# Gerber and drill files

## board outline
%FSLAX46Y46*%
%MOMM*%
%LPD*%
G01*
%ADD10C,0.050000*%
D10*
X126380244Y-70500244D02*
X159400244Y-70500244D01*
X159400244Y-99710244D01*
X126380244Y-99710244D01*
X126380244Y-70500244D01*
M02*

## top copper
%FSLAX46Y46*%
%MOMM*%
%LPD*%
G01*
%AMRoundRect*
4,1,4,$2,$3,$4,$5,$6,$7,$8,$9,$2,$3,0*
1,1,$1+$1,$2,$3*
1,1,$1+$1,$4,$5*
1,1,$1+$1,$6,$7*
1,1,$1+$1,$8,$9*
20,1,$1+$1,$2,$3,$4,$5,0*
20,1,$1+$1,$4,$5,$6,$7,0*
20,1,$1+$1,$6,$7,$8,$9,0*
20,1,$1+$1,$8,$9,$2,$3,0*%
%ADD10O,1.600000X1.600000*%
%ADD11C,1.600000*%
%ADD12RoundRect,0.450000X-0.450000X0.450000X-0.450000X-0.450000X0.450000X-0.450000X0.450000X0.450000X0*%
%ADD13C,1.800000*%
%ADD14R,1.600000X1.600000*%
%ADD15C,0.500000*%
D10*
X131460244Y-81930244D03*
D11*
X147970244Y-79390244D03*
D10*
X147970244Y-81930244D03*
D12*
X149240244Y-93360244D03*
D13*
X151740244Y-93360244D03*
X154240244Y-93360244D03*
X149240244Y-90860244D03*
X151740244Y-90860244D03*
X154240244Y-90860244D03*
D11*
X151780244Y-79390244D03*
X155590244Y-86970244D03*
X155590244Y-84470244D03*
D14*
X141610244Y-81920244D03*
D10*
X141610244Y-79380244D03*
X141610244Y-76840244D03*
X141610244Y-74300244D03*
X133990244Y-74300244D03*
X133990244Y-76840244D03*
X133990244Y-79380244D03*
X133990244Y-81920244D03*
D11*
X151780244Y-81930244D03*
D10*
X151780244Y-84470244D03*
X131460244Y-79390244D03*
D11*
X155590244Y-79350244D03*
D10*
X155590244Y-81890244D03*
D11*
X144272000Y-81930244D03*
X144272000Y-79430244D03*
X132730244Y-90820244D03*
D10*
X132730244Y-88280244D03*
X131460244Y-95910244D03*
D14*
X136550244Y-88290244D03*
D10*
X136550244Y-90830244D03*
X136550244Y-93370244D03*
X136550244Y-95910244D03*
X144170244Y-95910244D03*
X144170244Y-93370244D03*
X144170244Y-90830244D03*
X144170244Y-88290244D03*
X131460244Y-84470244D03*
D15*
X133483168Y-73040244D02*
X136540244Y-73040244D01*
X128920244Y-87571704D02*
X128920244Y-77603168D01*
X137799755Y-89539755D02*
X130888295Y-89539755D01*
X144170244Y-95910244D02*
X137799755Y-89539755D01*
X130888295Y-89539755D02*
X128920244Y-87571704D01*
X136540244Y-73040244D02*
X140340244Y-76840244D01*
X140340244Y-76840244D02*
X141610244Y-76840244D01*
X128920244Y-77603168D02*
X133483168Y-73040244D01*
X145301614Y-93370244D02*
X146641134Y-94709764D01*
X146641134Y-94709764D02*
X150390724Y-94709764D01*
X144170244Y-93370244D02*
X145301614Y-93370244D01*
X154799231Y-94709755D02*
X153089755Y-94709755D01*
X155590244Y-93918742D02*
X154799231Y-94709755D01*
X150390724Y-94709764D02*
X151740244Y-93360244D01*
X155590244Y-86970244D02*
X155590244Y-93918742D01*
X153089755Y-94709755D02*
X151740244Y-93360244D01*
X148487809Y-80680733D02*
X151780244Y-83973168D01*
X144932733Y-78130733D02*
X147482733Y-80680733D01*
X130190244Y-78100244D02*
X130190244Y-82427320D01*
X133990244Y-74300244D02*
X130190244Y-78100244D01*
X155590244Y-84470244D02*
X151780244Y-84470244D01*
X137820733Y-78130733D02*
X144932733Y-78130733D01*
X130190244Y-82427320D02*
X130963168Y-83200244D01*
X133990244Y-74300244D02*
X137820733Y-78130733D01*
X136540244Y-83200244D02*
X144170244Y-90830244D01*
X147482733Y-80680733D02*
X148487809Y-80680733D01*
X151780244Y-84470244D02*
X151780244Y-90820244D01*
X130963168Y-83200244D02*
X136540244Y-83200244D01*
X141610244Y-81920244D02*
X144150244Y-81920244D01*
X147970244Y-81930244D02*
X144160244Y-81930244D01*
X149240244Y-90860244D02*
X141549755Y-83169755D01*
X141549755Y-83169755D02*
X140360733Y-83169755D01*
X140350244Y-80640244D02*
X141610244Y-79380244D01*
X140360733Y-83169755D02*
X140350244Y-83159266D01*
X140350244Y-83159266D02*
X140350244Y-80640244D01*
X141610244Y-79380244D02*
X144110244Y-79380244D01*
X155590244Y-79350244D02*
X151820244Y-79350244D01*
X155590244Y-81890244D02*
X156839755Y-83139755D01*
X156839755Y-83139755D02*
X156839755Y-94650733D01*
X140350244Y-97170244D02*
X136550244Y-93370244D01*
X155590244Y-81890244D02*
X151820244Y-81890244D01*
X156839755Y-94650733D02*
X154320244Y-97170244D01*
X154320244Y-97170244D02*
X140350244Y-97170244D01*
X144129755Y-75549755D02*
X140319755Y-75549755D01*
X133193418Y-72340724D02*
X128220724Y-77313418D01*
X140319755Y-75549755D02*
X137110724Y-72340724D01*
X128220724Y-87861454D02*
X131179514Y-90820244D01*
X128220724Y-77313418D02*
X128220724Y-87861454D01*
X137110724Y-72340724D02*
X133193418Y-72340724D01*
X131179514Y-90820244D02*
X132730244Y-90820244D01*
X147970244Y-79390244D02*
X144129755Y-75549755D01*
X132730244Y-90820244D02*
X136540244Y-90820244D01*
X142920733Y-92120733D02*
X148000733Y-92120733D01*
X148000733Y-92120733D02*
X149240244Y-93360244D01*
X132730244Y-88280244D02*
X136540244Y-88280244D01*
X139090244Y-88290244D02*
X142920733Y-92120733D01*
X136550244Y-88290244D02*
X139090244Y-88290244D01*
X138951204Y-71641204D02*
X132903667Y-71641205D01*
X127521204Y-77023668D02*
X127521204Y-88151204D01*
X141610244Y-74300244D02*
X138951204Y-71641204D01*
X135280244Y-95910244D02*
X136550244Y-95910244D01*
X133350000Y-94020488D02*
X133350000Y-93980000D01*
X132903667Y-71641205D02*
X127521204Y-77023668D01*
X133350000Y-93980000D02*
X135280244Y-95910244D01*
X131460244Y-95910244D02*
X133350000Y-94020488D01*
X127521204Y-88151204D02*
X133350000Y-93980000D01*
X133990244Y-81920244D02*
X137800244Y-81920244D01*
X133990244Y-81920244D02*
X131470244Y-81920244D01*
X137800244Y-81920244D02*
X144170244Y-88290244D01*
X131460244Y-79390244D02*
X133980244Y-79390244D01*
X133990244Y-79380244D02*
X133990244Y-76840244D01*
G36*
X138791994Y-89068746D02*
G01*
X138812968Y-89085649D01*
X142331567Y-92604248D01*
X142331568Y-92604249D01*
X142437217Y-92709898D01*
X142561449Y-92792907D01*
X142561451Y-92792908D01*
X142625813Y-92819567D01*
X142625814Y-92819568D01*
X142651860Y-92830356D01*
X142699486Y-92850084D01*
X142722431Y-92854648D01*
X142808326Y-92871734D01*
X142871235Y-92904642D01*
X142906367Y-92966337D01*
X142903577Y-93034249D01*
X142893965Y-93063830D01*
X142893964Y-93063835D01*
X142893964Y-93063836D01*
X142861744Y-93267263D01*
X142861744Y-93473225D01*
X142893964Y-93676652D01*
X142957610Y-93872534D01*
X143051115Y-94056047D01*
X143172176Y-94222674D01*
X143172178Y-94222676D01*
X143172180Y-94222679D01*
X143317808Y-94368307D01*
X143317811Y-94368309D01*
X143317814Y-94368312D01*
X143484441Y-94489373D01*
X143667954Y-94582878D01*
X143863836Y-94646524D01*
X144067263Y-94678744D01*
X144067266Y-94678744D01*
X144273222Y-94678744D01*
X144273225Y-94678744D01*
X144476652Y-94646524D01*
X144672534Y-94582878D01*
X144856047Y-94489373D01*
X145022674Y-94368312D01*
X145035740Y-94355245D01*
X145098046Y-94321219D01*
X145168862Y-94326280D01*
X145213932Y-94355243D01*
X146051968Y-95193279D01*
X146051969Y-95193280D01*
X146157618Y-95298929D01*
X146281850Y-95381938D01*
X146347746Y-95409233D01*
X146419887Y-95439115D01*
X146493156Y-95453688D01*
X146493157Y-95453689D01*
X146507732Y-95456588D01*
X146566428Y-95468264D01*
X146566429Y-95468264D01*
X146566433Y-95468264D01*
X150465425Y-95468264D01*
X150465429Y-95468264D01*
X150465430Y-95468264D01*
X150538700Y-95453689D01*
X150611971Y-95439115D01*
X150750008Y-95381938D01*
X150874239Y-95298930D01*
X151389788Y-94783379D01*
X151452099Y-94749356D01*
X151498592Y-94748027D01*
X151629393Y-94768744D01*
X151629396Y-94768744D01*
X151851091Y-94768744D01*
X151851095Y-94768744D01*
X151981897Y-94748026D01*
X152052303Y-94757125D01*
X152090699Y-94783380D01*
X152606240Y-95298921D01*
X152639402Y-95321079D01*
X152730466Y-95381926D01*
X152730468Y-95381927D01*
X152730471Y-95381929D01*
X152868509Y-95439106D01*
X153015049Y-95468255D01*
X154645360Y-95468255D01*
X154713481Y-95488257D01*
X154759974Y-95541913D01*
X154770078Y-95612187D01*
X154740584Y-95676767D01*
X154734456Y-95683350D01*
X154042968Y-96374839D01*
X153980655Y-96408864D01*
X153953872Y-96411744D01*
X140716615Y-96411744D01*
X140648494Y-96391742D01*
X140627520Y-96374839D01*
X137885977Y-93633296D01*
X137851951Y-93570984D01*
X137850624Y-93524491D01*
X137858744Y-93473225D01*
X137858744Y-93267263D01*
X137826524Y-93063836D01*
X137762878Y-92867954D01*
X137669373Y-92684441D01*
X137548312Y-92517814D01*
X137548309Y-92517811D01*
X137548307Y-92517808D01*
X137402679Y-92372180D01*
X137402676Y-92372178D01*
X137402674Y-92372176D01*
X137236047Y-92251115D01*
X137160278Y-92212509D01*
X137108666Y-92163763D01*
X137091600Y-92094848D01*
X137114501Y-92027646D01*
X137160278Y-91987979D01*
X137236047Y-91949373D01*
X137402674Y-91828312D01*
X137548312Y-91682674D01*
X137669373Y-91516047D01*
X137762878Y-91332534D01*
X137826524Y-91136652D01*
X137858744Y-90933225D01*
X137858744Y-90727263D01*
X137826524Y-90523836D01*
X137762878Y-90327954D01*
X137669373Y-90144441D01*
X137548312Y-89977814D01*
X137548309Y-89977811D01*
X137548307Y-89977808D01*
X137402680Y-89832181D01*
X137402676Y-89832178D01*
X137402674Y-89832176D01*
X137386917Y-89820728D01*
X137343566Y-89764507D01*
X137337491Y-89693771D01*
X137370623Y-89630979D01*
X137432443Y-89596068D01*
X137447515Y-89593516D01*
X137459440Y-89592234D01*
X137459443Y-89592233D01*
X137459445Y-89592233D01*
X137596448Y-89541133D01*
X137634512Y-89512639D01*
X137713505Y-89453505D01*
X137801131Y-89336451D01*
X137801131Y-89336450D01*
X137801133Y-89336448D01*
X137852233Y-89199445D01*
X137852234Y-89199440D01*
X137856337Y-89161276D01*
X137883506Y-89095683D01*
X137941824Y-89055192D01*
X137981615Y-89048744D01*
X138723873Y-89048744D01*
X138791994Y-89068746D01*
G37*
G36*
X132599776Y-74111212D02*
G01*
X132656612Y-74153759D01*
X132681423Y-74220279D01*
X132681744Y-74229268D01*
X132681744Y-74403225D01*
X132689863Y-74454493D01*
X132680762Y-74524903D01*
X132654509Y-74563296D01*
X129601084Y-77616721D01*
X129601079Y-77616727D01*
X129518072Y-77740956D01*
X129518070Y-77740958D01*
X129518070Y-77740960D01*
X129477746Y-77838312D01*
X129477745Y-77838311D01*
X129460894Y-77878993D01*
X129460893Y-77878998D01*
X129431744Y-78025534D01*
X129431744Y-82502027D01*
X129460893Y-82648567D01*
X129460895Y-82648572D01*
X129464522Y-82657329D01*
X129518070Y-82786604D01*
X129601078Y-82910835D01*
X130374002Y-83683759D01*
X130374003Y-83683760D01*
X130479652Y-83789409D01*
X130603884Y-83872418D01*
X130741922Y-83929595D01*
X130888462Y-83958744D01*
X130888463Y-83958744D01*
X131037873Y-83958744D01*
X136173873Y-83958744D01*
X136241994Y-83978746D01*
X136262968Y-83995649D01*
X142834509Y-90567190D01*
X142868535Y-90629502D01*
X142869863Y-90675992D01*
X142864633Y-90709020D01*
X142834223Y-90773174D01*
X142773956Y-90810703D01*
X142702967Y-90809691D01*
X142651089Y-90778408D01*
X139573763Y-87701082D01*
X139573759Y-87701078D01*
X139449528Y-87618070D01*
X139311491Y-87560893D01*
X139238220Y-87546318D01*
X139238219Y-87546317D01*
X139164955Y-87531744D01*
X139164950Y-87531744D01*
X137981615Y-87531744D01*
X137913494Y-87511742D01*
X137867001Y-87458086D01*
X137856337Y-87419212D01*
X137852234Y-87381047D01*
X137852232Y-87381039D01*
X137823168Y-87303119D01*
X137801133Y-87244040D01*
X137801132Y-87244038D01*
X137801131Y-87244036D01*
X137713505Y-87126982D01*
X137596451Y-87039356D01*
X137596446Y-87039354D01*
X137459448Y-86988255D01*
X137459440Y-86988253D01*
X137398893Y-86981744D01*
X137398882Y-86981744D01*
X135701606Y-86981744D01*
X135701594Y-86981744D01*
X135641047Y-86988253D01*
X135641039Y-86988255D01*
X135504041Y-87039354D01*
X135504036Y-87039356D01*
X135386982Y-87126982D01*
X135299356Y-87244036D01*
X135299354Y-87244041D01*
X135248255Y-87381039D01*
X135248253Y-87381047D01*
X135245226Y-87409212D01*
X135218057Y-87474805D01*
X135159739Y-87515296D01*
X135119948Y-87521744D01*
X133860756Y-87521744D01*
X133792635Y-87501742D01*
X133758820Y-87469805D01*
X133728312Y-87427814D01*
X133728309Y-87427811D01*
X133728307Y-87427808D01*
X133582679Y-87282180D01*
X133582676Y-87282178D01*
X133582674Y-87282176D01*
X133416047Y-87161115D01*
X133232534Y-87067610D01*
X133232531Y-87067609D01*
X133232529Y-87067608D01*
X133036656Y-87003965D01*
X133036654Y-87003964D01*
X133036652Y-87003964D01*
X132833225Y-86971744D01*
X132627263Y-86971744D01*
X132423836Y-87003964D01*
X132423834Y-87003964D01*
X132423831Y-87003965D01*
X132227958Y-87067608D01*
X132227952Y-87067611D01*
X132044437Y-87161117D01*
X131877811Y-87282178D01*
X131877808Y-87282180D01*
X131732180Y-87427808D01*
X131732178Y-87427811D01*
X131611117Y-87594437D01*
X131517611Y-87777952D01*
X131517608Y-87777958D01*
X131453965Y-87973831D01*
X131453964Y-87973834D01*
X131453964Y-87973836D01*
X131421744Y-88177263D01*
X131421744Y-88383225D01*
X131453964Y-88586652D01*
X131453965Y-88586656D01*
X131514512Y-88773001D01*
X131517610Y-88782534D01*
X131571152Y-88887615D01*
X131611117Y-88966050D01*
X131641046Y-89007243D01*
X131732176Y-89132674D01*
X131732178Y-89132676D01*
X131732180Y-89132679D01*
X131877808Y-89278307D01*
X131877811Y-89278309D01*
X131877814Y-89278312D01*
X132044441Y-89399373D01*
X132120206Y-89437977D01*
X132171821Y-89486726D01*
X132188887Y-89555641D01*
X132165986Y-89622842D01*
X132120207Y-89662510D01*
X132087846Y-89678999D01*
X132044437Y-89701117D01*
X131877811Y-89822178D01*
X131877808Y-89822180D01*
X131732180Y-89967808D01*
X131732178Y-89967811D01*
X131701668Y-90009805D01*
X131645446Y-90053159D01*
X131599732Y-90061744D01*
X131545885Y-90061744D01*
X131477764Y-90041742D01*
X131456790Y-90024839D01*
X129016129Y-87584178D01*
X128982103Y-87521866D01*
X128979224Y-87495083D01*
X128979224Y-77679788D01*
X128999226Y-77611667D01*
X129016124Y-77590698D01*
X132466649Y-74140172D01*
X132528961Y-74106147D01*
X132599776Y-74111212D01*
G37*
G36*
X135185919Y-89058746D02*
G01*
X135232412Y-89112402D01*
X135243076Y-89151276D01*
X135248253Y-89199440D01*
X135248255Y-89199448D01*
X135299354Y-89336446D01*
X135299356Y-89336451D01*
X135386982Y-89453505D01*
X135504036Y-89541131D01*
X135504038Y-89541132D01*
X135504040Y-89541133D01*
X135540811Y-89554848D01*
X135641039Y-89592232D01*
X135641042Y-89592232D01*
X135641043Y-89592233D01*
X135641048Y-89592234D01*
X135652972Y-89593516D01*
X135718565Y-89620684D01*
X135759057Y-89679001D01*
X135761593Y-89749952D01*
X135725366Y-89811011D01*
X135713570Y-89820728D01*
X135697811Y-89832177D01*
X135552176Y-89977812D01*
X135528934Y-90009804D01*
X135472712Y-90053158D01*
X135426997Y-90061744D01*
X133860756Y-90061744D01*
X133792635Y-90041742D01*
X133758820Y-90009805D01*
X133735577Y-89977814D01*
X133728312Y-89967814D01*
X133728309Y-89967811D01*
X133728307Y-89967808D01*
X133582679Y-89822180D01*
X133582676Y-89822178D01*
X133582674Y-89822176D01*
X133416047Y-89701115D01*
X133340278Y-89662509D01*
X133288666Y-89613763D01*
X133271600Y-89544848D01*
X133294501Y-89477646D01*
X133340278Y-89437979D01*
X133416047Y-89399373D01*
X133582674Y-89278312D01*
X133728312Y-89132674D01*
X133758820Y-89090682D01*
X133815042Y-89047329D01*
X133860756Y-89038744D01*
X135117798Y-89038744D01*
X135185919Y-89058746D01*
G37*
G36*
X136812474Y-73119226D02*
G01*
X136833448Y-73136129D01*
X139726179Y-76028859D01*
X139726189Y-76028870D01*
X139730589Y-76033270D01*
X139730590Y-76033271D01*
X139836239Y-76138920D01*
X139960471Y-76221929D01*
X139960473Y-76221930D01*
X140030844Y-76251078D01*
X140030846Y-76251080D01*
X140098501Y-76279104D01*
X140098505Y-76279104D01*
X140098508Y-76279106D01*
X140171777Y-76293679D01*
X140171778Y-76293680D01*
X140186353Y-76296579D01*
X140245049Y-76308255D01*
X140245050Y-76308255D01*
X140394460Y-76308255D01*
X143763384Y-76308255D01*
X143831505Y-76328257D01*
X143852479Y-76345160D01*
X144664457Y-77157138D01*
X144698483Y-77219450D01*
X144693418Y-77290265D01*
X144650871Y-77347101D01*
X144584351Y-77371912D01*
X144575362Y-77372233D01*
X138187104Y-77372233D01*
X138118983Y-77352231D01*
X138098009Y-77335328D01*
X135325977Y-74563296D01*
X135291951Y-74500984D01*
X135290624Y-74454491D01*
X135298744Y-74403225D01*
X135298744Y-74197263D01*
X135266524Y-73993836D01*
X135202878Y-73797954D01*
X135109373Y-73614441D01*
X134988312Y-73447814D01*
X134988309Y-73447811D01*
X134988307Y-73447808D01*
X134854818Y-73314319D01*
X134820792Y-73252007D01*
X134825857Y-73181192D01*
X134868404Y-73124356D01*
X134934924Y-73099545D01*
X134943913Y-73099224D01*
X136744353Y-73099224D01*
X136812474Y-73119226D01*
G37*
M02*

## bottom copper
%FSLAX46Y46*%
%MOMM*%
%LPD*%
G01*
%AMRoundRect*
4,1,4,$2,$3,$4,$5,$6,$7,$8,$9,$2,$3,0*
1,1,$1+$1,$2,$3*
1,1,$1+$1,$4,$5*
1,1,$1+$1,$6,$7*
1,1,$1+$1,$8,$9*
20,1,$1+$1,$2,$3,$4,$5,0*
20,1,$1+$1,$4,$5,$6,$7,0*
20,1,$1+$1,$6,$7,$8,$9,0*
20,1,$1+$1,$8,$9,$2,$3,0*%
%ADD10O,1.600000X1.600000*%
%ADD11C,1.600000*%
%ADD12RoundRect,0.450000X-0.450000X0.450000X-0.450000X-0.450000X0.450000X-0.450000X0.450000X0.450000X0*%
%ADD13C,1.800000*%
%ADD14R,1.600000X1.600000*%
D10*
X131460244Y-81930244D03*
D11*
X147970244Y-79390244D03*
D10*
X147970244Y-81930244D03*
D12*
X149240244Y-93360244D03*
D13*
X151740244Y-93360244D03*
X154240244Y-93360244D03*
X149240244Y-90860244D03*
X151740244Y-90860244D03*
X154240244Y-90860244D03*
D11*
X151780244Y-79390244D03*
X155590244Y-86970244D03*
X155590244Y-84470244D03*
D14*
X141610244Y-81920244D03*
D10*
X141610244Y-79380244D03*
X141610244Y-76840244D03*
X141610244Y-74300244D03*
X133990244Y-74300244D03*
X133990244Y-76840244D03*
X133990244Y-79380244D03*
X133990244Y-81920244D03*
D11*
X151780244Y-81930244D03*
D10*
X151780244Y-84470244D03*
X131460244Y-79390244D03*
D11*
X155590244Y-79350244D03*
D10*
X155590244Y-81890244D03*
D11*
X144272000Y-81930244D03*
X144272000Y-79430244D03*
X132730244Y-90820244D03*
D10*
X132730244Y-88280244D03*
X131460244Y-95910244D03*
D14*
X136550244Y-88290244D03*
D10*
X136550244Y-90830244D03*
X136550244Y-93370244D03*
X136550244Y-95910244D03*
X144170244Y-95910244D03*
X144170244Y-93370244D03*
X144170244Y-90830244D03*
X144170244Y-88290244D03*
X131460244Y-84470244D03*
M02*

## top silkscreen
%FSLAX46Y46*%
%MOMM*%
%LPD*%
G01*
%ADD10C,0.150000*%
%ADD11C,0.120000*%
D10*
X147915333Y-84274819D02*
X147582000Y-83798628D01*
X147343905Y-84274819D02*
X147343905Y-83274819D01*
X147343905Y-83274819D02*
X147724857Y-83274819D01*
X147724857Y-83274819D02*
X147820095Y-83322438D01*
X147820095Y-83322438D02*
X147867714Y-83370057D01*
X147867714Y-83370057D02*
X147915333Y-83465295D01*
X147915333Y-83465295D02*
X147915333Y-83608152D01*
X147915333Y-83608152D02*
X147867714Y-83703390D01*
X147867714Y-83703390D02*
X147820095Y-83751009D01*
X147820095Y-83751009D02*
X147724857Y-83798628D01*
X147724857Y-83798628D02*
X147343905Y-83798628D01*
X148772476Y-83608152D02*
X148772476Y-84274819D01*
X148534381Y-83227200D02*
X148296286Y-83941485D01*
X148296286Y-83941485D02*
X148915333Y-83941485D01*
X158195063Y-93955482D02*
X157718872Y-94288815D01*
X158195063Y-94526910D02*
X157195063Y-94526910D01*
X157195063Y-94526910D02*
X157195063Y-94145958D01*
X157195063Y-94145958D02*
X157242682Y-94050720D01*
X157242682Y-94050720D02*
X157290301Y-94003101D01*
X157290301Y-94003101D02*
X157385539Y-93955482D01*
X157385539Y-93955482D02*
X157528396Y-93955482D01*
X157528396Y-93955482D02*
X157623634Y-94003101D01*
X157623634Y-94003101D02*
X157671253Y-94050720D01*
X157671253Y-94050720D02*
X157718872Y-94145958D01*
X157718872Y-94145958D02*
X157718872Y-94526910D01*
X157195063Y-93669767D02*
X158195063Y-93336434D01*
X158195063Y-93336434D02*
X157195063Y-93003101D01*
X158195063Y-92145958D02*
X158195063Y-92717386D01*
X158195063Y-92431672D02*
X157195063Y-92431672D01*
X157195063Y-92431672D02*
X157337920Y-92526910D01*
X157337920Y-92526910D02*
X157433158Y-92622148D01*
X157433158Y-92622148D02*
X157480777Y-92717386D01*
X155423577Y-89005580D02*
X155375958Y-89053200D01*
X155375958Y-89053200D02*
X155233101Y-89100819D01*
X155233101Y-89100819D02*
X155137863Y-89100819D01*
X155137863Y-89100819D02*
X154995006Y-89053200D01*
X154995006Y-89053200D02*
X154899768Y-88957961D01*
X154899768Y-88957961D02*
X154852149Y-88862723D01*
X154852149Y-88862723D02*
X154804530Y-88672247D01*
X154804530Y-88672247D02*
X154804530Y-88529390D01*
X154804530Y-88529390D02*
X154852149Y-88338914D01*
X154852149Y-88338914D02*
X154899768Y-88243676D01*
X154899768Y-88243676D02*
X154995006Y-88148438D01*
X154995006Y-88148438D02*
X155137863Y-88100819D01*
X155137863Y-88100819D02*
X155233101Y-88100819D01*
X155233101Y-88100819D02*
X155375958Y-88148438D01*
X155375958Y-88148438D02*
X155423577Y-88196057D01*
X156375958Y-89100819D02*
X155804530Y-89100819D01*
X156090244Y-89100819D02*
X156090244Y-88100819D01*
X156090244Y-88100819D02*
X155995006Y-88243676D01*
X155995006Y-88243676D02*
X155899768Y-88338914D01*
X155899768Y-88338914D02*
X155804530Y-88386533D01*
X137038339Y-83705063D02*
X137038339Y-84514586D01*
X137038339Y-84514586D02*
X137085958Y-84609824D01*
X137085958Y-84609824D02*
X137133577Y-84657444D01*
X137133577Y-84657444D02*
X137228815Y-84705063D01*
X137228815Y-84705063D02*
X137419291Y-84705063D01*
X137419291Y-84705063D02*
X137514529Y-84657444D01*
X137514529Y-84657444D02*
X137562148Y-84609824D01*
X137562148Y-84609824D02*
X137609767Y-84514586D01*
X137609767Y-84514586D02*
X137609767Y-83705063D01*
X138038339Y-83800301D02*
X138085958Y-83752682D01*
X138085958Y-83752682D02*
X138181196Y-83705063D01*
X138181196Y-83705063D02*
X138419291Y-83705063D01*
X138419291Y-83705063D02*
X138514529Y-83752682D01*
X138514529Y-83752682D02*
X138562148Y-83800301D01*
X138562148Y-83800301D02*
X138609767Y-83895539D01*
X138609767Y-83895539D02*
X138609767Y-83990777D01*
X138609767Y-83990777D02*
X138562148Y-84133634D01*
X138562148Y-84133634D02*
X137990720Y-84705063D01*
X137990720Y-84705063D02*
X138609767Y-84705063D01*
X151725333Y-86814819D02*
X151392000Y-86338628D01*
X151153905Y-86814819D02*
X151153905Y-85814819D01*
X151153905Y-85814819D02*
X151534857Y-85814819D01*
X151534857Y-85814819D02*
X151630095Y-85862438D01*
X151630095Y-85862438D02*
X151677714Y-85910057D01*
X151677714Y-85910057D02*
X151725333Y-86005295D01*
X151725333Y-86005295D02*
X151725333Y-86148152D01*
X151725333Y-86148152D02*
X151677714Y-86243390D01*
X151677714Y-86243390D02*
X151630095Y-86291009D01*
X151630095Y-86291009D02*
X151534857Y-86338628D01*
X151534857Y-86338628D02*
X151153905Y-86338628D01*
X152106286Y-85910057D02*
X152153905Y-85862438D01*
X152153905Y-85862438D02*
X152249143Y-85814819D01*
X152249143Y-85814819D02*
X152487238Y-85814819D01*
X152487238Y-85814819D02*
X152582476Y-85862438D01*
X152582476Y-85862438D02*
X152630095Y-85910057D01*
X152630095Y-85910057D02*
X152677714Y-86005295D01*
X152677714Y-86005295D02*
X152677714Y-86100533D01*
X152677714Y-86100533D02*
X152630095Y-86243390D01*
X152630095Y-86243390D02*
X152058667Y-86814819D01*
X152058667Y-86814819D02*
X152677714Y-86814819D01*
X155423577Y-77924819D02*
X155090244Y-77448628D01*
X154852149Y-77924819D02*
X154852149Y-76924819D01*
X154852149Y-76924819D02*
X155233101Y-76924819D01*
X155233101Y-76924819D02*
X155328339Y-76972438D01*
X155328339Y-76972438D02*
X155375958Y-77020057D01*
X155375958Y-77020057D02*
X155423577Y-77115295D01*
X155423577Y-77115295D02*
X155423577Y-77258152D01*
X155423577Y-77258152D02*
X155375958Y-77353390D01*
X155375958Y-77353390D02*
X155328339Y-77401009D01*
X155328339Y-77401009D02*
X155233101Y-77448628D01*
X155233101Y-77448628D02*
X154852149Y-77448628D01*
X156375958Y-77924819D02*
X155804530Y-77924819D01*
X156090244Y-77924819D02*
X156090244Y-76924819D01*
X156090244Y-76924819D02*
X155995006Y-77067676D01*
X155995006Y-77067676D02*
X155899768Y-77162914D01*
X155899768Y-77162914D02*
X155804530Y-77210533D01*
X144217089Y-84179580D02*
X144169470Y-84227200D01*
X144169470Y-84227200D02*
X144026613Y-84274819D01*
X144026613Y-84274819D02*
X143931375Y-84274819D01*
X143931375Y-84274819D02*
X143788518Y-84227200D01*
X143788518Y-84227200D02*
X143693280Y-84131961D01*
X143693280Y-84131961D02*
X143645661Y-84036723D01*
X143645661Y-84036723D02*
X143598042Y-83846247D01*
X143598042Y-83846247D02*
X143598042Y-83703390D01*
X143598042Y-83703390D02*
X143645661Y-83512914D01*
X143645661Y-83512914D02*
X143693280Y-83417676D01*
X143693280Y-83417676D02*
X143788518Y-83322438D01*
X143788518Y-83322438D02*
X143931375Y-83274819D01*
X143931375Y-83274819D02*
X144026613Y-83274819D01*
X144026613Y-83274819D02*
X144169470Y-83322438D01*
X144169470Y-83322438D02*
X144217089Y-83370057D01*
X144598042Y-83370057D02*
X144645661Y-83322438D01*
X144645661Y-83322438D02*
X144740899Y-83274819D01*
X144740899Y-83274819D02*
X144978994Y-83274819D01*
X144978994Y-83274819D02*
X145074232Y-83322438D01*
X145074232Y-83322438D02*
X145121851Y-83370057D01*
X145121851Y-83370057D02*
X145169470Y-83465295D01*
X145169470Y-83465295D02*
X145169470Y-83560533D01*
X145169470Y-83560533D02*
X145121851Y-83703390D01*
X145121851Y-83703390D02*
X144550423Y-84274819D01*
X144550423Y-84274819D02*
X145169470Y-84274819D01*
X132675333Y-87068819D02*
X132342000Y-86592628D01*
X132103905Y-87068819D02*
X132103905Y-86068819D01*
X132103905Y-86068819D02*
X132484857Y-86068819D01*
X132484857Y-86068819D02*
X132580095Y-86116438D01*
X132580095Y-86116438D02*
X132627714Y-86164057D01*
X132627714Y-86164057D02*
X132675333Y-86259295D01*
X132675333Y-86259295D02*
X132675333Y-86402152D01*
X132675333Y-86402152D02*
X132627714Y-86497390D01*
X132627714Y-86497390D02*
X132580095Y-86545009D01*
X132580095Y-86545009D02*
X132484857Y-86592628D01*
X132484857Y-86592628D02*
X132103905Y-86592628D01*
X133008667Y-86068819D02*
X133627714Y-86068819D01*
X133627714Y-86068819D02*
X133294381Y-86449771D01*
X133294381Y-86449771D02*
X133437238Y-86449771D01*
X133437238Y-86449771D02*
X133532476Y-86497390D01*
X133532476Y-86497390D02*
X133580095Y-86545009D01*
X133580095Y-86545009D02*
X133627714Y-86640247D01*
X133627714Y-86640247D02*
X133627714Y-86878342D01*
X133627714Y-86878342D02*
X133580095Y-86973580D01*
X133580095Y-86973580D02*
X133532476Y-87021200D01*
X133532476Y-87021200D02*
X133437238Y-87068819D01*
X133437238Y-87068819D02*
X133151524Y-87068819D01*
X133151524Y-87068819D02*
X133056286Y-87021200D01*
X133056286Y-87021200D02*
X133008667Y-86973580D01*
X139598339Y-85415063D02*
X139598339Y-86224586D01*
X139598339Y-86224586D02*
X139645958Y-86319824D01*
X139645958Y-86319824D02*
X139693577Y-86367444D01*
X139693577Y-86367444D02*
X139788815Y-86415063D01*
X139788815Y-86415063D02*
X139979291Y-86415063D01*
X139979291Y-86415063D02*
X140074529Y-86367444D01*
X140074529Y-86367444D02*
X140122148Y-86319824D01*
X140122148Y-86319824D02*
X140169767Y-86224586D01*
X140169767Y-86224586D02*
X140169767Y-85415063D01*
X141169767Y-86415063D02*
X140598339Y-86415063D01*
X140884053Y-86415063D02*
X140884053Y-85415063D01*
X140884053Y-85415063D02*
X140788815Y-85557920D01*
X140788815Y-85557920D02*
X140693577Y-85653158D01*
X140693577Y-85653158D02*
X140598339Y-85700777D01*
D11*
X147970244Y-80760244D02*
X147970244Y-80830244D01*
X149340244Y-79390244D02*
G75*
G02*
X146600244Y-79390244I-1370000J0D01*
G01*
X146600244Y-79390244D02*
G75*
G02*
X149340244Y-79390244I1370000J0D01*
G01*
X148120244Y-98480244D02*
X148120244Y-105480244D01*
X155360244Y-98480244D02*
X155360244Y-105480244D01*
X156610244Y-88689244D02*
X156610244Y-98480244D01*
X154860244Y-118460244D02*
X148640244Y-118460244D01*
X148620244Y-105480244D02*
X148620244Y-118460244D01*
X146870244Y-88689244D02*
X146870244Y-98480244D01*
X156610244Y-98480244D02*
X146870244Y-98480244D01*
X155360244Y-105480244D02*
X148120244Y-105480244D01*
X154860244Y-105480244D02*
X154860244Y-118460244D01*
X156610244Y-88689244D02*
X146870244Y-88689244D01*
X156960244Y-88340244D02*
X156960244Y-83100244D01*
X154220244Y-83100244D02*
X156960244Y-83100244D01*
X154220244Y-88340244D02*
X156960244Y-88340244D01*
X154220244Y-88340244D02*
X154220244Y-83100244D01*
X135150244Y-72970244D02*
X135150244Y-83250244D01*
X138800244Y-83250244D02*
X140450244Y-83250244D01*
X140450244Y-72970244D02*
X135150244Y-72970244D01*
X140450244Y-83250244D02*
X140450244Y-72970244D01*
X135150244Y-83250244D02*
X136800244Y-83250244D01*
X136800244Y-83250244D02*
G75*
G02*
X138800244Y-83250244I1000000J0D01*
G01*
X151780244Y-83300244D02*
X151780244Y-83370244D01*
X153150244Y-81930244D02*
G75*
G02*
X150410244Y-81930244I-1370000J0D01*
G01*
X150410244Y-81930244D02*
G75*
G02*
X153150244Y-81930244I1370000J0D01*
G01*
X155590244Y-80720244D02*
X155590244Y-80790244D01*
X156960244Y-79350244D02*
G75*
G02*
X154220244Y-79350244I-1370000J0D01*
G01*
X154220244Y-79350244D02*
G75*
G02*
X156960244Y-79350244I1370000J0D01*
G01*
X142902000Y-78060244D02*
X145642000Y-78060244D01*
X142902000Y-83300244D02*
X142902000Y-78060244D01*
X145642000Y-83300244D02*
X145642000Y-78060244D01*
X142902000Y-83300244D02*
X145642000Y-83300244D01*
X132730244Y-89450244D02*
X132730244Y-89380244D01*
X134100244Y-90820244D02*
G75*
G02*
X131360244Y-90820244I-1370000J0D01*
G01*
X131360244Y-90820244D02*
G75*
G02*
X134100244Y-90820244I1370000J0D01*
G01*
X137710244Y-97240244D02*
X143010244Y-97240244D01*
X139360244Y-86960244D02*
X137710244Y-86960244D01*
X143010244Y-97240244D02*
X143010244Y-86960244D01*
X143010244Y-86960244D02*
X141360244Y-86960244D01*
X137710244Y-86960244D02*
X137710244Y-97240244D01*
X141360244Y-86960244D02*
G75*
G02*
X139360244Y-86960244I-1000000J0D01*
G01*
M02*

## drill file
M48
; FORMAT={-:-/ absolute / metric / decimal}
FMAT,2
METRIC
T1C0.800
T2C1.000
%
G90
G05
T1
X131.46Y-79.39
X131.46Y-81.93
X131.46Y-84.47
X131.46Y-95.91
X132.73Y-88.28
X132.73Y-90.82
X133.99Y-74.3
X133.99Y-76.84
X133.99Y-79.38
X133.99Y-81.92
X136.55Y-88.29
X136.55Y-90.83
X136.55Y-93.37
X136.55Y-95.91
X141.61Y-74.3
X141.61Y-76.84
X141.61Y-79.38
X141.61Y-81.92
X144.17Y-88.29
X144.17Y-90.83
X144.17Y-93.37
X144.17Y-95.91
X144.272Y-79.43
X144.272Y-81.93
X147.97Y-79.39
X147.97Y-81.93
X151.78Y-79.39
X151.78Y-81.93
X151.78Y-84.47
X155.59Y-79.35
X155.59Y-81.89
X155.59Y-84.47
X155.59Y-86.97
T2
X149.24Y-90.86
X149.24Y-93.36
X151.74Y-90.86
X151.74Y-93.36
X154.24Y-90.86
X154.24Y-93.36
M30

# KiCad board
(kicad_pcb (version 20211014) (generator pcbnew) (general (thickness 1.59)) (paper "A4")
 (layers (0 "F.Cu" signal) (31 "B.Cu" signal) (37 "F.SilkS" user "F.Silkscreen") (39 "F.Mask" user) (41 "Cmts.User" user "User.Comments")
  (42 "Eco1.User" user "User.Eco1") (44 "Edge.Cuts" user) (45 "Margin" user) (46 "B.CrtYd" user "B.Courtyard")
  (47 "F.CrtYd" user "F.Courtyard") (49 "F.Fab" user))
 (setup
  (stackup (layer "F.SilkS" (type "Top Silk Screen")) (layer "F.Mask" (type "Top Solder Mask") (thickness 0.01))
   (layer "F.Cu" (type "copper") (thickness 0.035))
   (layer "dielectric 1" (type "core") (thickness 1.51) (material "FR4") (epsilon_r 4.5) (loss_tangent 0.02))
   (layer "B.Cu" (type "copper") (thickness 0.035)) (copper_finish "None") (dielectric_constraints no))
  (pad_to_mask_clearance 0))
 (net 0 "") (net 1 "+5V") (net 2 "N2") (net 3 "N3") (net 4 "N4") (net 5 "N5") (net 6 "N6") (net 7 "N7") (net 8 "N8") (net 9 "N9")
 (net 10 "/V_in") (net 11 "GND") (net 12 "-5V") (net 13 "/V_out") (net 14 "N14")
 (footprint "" (layer "F.Cu") (at 131.460244 81.930244)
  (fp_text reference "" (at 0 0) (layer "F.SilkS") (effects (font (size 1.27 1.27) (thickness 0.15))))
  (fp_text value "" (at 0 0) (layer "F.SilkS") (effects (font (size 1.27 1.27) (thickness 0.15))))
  (pad "8" thru_hole oval (at 0 0) (size 1.6 1.6) (drill 0.8) (layers *.Cu *.Mask) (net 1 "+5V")))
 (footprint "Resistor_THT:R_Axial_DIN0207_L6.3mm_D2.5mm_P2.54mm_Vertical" (layer "F.Cu") (at 147.970244 79.390244 -90)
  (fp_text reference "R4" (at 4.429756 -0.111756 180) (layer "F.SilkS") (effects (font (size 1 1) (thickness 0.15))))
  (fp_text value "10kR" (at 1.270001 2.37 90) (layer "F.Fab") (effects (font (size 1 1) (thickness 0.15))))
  (fp_line (start 1.37 0) (end 1.44 0) (layer "F.SilkS") (width 0.12))
  (fp_circle (center 0 0) (end 1.37 0) (layer "F.SilkS") (width 0.12) (fill none))
  (pad "1" thru_hole circle (at 0 0 270) (size 1.6 1.6) (drill 0.8) (layers *.Cu *.Mask) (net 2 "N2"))
  (pad "2" thru_hole oval (at 2.54 0 270) (size 1.6 1.6) (drill 0.8) (layers *.Cu *.Mask) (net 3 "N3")))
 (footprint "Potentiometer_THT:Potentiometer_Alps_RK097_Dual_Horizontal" (layer "F.Cu") (at 149.240244 93.360244 90)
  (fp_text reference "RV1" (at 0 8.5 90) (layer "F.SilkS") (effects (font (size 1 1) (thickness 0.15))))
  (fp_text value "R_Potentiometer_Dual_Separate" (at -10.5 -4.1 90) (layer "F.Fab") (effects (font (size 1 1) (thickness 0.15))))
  (fp_line (start -5.12 -1.12) (end -12.12 -1.12) (layer "F.SilkS") (width 0.12))
  (fp_line (start -5.12 6.12) (end -12.12 6.12) (layer "F.SilkS") (width 0.12))
  (fp_line (start 4.671 7.37) (end -5.12 7.37) (layer "F.SilkS") (width 0.12))
  (fp_line (start -25.1 5.62) (end -25.1 -0.6) (layer "F.SilkS") (width 0.12))
  (fp_line (start -12.12 -0.62) (end -25.1 -0.62) (layer "F.SilkS") (width 0.12))
  (fp_line (start 4.671 -2.37) (end -5.12 -2.37) (layer "F.SilkS") (width 0.12))
  (fp_line (start -5.12 7.37) (end -5.12 -2.37) (layer "F.SilkS") (width 0.12))
  (fp_line (start -12.12 6.12) (end -12.12 -1.12) (layer "F.SilkS") (width 0.12))
  (fp_line (start -12.12 5.62) (end -25.1 5.62) (layer "F.SilkS") (width 0.12))
  (fp_line (start 4.671 7.37) (end 4.671 -2.37) (layer "F.SilkS") (width 0.12))
  (pad "1" thru_hole roundrect (at 0 0 270) (size 1.8 1.8) (drill 1) (layers *.Cu *.Mask) (roundrect_rratio 0.25) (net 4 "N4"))
  (pad "2" thru_hole circle (at 0 2.5 270) (size 1.8 1.8) (drill 1) (layers *.Cu *.Mask) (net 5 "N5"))
  (pad "3" thru_hole circle (at 0 5 270) (size 1.8 1.8) (drill 1) (layers *.Cu *.Mask) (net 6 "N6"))
  (pad "4" thru_hole circle (at 2.5 0 270) (size 1.8 1.8) (drill 1) (layers *.Cu *.Mask) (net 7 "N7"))
  (pad "5" thru_hole circle (at 2.5 2.5 270) (size 1.8 1.8) (drill 1) (layers *.Cu *.Mask) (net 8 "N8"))
  (pad "6" thru_hole circle (at 2.5 5 270) (size 1.8 1.8) (drill 1) (layers *.Cu *.Mask) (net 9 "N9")))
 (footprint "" (layer "F.Cu") (at 151.780244 79.390244)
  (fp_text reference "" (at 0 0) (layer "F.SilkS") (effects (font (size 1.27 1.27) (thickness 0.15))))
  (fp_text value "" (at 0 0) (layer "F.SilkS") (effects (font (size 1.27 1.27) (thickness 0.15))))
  (pad "1" thru_hole circle (at 0 0 270) (size 1.6 1.6) (drill 0.8) (layers *.Cu *.Mask) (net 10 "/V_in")))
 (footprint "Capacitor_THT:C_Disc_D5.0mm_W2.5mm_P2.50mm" (layer "F.Cu") (at 155.590244 86.970244 90)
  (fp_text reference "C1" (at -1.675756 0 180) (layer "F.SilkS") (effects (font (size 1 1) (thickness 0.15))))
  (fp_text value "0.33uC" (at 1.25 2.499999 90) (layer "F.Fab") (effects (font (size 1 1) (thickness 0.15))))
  (fp_line (start -1.37 1.37) (end 3.87 1.37) (layer "F.SilkS") (width 0.12))
  (fp_line (start 3.87 -1.37) (end 3.87 1.37) (layer "F.SilkS") (width 0.12))
  (fp_line (start -1.37 -1.37) (end -1.37 1.37) (layer "F.SilkS") (width 0.12))
  (fp_line (start -1.37 -1.37) (end 3.87 -1.37) (layer "F.SilkS") (width 0.12))
  (pad "1" thru_hole circle (at 0 0 90) (size 1.6 1.6) (drill 0.8) (layers *.Cu *.Mask) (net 5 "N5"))
  (pad "2" thru_hole circle (at 2.5 0 90) (size 1.6 1.6) (drill 0.8) (layers *.Cu *.Mask) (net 8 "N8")))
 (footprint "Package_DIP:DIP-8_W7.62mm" (layer "F.Cu") (at 141.610244 81.920244 180)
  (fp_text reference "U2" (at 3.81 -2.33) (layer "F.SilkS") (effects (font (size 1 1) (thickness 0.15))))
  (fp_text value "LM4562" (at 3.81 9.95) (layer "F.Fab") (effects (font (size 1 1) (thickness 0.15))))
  (fp_line (start 6.46 8.95) (end 6.46 -1.33) (layer "F.SilkS") (width 0.12))
  (fp_line (start 2.81 -1.33) (end 1.16 -1.33) (layer "F.SilkS") (width 0.12))
  (fp_line (start 1.16 8.95) (end 6.46 8.95) (layer "F.SilkS") (width 0.12))
  (fp_line (start 1.16 -1.33) (end 1.16 8.95) (layer "F.SilkS") (width 0.12))
  (fp_line (start 6.46 -1.33) (end 4.81 -1.33) (layer "F.SilkS") (width 0.12))
  (fp_arc (start 4.81 -1.33) (mid 3.81 -0.33) (end 2.81 -1.33) (layer "F.SilkS") (width 0.12))
  (pad "1" thru_hole rect (at 0 0 180) (size 1.6 1.6) (drill 0.8) (layers *.Cu *.Mask) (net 3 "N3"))
  (pad "2" thru_hole oval (at 0 2.54 180) (size 1.6 1.6) (drill 0.8) (layers *.Cu *.Mask) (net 7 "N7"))
  (pad "3" thru_hole oval (at 0 5.08 180) (size 1.6 1.6) (drill 0.8) (layers *.Cu *.Mask) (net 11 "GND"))
  (pad "4" thru_hole oval (at 0 7.62 180) (size 1.6 1.6) (drill 0.8) (layers *.Cu *.Mask) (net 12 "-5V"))
  (pad "5" thru_hole oval (at 7.62 7.62 180) (size 1.6 1.6) (drill 0.8) (layers *.Cu *.Mask) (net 8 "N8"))
  (pad "6" thru_hole oval (at 7.62 5.08 180) (size 1.6 1.6) (drill 0.8) (layers *.Cu *.Mask) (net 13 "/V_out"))
  (pad "7" thru_hole oval (at 7.62 2.54 180) (size 1.6 1.6) (drill 0.8) (layers *.Cu *.Mask) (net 13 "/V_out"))
  (pad "8" thru_hole oval (at 7.62 0 180) (size 1.6 1.6) (drill 0.8) (layers *.Cu *.Mask) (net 1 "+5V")))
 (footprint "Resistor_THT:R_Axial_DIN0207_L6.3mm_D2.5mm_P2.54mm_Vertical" (layer "F.Cu") (at 151.780244 81.930244 -90)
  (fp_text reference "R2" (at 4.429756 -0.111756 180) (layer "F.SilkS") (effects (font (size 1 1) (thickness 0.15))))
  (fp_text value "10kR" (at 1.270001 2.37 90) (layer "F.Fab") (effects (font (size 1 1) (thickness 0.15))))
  (fp_line (start 1.37 0) (end 1.44 0) (layer "F.SilkS") (width 0.12))
  (fp_circle (center 0 0) (end 1.37 0) (layer "F.SilkS") (width 0.12) (fill none))
  (pad "1" thru_hole circle (at 0 0 270) (size 1.6 1.6) (drill 0.8) (layers *.Cu *.Mask) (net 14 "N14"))
  (pad "2" thru_hole oval (at 2.54 0 270) (size 1.6 1.6) (drill 0.8) (layers *.Cu *.Mask) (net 8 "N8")))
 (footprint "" (layer "F.Cu") (at 131.460244 79.390244)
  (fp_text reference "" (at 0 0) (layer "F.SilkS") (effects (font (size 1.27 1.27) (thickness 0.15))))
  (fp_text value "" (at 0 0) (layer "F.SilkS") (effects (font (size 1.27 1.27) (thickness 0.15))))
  (pad "7" thru_hole oval (at 0 0 180) (size 1.6 1.6) (drill 0.8) (layers *.Cu *.Mask) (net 13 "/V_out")))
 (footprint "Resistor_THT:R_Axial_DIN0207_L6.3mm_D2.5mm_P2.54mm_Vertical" (layer "F.Cu") (at 155.590244 79.350244 -90)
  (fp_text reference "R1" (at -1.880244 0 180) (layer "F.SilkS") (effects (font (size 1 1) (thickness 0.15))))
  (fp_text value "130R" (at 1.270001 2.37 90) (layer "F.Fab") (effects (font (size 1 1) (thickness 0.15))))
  (fp_line (start 1.37 0) (end 1.44 0) (layer "F.SilkS") (width 0.12))
  (fp_circle (center 0 0) (end 1.37 0) (layer "F.SilkS") (width 0.12) (fill none))
  (pad "1" thru_hole circle (at 0 0 270) (size 1.6 1.6) (drill 0.8) (layers *.Cu *.Mask) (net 10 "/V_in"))
  (pad "2" thru_hole oval (at 2.54 0 270) (size 1.6 1.6) (drill 0.8) (layers *.Cu *.Mask) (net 14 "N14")))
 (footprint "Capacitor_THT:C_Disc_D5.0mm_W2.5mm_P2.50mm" (layer "F.Cu") (at 144.272 81.930244 90)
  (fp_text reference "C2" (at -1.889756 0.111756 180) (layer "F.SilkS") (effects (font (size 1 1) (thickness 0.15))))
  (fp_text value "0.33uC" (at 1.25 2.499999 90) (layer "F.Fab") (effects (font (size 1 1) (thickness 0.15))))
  (fp_line (start 3.87 -1.37) (end 3.87 1.37) (layer "F.SilkS") (width 0.12))
  (fp_line (start -1.37 -1.37) (end 3.87 -1.37) (layer "F.SilkS") (width 0.12))
  (fp_line (start -1.37 1.37) (end 3.87 1.37) (layer "F.SilkS") (width 0.12))
  (fp_line (start -1.37 -1.37) (end -1.37 1.37) (layer "F.SilkS") (width 0.12))
  (pad "1" thru_hole circle (at 0 0 90) (size 1.6 1.6) (drill 0.8) (layers *.Cu *.Mask) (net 3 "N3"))
  (pad "2" thru_hole circle (at 2.5 0 90) (size 1.6 1.6) (drill 0.8) (layers *.Cu *.Mask) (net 7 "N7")))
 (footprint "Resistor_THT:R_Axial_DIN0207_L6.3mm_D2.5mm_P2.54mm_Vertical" (layer "F.Cu") (at 132.730244 90.820244 90)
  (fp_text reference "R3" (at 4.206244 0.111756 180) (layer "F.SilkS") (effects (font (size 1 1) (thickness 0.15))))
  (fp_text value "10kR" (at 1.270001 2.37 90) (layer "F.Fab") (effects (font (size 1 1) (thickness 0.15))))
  (fp_line (start 1.37 0) (end 1.44 0) (layer "F.SilkS") (width 0.12))
  (fp_circle (center 0 0) (end 1.37 0) (layer "F.SilkS") (width 0.12) (fill none))
  (pad "1" thru_hole circle (at 0 0 90) (size 1.6 1.6) (drill 0.8) (layers *.Cu *.Mask) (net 2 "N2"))
  (pad "2" thru_hole oval (at 2.54 0 90) (size 1.6 1.6) (drill 0.8) (layers *.Cu *.Mask) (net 4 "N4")))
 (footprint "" (layer "F.Cu") (at 131.360244 95.758)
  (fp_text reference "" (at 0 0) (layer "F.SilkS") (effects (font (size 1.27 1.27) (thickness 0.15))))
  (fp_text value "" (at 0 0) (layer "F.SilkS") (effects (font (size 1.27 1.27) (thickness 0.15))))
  (pad "4" thru_hole oval (at 0.1 0.152244) (size 1.6 1.6) (drill 0.8) (layers *.Cu "F.Mask") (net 12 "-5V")))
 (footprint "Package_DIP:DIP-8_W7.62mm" (layer "F.Cu") (at 136.550244 88.290244)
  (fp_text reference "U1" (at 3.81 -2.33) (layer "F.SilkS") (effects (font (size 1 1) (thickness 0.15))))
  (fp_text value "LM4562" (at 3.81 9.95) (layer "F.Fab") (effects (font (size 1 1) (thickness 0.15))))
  (fp_line (start 1.16 8.95) (end 6.46 8.95) (layer "F.SilkS") (width 0.12))
  (fp_line (start 2.81 -1.33) (end 1.16 -1.33) (layer "F.SilkS") (width 0.12))
  (fp_line (start 6.46 8.95) (end 6.46 -1.33) (layer "F.SilkS") (width 0.12))
  (fp_line (start 6.46 -1.33) (end 4.81 -1.33) (layer "F.SilkS") (width 0.12))
  (fp_line (start 1.16 -1.33) (end 1.16 8.95) (layer "F.SilkS") (width 0.12))
  (fp_arc (start 4.81 -1.33) (mid 3.81 -0.33) (end 2.81 -1.33) (layer "F.SilkS") (width 0.12))
  (pad "1" thru_hole rect (at 0 0) (size 1.6 1.6) (drill 0.8) (layers *.Cu *.Mask) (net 4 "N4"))
  (pad "2" thru_hole oval (at 0 2.54) (size 1.6 1.6) (drill 0.8) (layers *.Cu *.Mask) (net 2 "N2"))
  (pad "3" thru_hole oval (at 0 5.08) (size 1.6 1.6) (drill 0.8) (layers *.Cu *.Mask) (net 14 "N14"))
  (pad "4" thru_hole oval (at 0 7.62) (size 1.6 1.6) (drill 0.8) (layers *.Cu *.Mask) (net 12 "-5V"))
  (pad "5" thru_hole oval (at 7.62 7.62) (size 1.6 1.6) (drill 0.8) (layers *.Cu *.Mask) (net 11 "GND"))
  (pad "6" thru_hole oval (at 7.62 5.08) (size 1.6 1.6) (drill 0.8) (layers *.Cu *.Mask) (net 5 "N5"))
  (pad "7" thru_hole oval (at 7.62 2.54) (size 1.6 1.6) (drill 0.8) (layers *.Cu *.Mask) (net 8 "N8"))
  (pad "8" thru_hole oval (at 7.62 0) (size 1.6 1.6) (drill 0.8) (layers *.Cu *.Mask) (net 1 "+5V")))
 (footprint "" (layer "F.Cu") (at 131.460244 84.470244)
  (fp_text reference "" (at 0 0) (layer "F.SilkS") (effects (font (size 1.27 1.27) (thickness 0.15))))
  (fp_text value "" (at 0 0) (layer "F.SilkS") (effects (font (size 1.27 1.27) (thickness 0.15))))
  (pad "5" thru_hole oval (at 0 0) (size 1.6 1.6) (drill 0.8) (layers *.Cu *.Mask) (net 11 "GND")))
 (gr_rect (start 159.400244 99.710244) (end 126.380244 70.500244) (layer "Edge.Cuts") (width 0.05) (fill none))
 (segment (start 133.483168 73.040244) (end 136.540244 73.040244) (width 0.5) (layer "F.Cu") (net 11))
 (segment (start 128.920244 87.571704) (end 128.920244 77.603168) (width 0.5) (layer "F.Cu") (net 11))
 (segment (start 137.799755 89.539755) (end 130.888295 89.539755) (width 0.5) (layer "F.Cu") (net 11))
 (segment (start 144.170244 95.910244) (end 137.799755 89.539755) (width 0.5) (layer "F.Cu") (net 11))
 (segment (start 130.888295 89.539755) (end 128.920244 87.571704) (width 0.5) (layer "F.Cu") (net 11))
 (segment (start 136.540244 73.040244) (end 140.340244 76.840244) (width 0.5) (layer "F.Cu") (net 11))
 (segment (start 140.340244 76.840244) (end 141.610244 76.840244) (width 0.5) (layer "F.Cu") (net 11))
 (segment (start 128.920244 77.603168) (end 133.483168 73.040244) (width 0.5) (layer "F.Cu") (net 11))
 (segment (start 145.301614 93.370244) (end 146.641134 94.709764) (width 0.5) (layer "F.Cu") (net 5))
 (segment (start 146.641134 94.709764) (end 150.390724 94.709764) (width 0.5) (layer "F.Cu") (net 5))
 (segment (start 144.170244 93.370244) (end 145.301614 93.370244) (width 0.5) (layer "F.Cu") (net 5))
 (segment (start 154.799231 94.709755) (end 153.089755 94.709755) (width 0.5) (layer "F.Cu") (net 5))
 (segment (start 155.590244 93.918742) (end 154.799231 94.709755) (width 0.5) (layer "F.Cu") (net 5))
 (segment (start 150.390724 94.709764) (end 151.740244 93.360244) (width 0.5) (layer "F.Cu") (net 5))
 (segment (start 155.590244 86.970244) (end 155.590244 93.918742) (width 0.5) (layer "F.Cu") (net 5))
 (segment (start 153.089755 94.709755) (end 151.740244 93.360244) (width 0.5) (layer "F.Cu") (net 5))
 (segment (start 148.487809 80.680733) (end 151.780244 83.973168) (width 0.5) (layer "F.Cu") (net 8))
 (segment (start 144.932733 78.130733) (end 147.482733 80.680733) (width 0.5) (layer "F.Cu") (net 8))
 (segment (start 130.190244 78.100244) (end 130.190244 82.42732) (width 0.5) (layer "F.Cu") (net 8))
 (segment (start 133.990244 74.300244) (end 130.190244 78.100244) (width 0.5) (layer "F.Cu") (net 8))
 (segment (start 155.590244 84.470244) (end 151.780244 84.470244) (width 0.5) (layer "F.Cu") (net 8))
 (segment (start 137.820733 78.130733) (end 144.932733 78.130733) (width 0.5) (layer "F.Cu") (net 8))
 (segment (start 130.190244 82.42732) (end 130.963168 83.200244) (width 0.5) (layer "F.Cu") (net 8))
 (segment (start 133.990244 74.300244) (end 137.820733 78.130733) (width 0.5) (layer "F.Cu") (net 8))
 (segment (start 136.540244 83.200244) (end 144.170244 90.830244) (width 0.5) (layer "F.Cu") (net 8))
 (segment (start 147.482733 80.680733) (end 148.487809 80.680733) (width 0.5) (layer "F.Cu") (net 8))
 (segment (start 151.780244 84.470244) (end 151.780244 90.820244) (width 0.5) (layer "F.Cu") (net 8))
 (segment (start 130.963168 83.200244) (end 136.540244 83.200244) (width 0.5) (layer "F.Cu") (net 8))
 (segment (start 141.610244 81.920244) (end 144.150244 81.920244) (width 0.5) (layer "F.Cu") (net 3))
 (segment (start 147.970244 81.930244) (end 144.160244 81.930244) (width 0.5) (layer "F.Cu") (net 3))
 (segment (start 149.240244 90.860244) (end 141.549755 83.169755) (width 0.5) (layer "F.Cu") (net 7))
 (segment (start 141.549755 83.169755) (end 140.360733 83.169755) (width 0.5) (layer "F.Cu") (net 7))
 (segment (start 140.350244 80.640244) (end 141.610244 79.380244) (width 0.5) (layer "F.Cu") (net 7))
 (segment (start 140.360733 83.169755) (end 140.350244 83.159266) (width 0.5) (layer "F.Cu") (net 7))
 (segment (start 140.350244 83.159266) (end 140.350244 80.640244) (width 0.5) (layer "F.Cu") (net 7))
 (segment (start 141.610244 79.380244) (end 144.110244 79.380244) (width 0.5) (layer "F.Cu") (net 7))
 (segment (start 155.590244 79.350244) (end 151.820244 79.350244) (width 0.5) (layer "F.Cu") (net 10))
 (segment (start 155.590244 81.890244) (end 156.839755 83.139755) (width 0.5) (layer "F.Cu") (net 14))
 (segment (start 156.839755 83.139755) (end 156.839755 94.650733) (width 0.5) (layer "F.Cu") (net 14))
 (segment (start 140.350244 97.170244) (end 136.550244 93.370244) (width 0.5) (layer "F.Cu") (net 14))
 (segment (start 155.590244 81.890244) (end 151.820244 81.890244) (width 0.5) (layer "F.Cu") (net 14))
 (segment (start 156.839755 94.650733) (end 154.320244 97.170244) (width 0.5) (layer "F.Cu") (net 14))
 (segment (start 154.320244 97.170244) (end 140.350244 97.170244) (width 0.5) (layer "F.Cu") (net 14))
 (segment (start 144.129755 75.549755) (end 140.319755 75.549755) (width 0.5) (layer "F.Cu") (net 2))
 (segment (start 133.193418 72.340724) (end 128.220724 77.313418) (width 0.5) (layer "F.Cu") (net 2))
 (segment (start 140.319755 75.549755) (end 137.110724 72.340724) (width 0.5) (layer "F.Cu") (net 2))
 (segment (start 128.220724 87.861454) (end 131.179514 90.820244) (width 0.5) (layer "F.Cu") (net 2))
 (segment (start 128.220724 77.313418) (end 128.220724 87.861454) (width 0.5) (layer "F.Cu") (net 2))
 (segment (start 137.110724 72.340724) (end 133.193418 72.340724) (width 0.5) (layer "F.Cu") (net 2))
 (segment (start 131.179514 90.820244) (end 132.730244 90.820244) (width 0.5) (layer "F.Cu") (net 2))
 (segment (start 147.970244 79.390244) (end 144.129755 75.549755) (width 0.5) (layer "F.Cu") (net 2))
 (segment (start 132.730244 90.820244) (end 136.540244 90.820244) (width 0.5) (layer "F.Cu") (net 2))
 (segment (start 142.920733 92.120733) (end 148.000733 92.120733) (width 0.5) (layer "F.Cu") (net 4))
 (segment (start 148.000733 92.120733) (end 149.240244 93.360244) (width 0.5) (layer "F.Cu") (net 4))
 (segment (start 132.730244 88.280244) (end 136.540244 88.280244) (width 0.5) (layer "F.Cu") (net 4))
 (segment (start 139.090244 88.290244) (end 142.920733 92.120733) (width 0.5) (layer "F.Cu") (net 4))
 (segment (start 136.550244 88.290244) (end 139.090244 88.290244) (width 0.5) (layer "F.Cu") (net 4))
 (segment (start 138.951204 71.641204) (end 132.903667 71.641205) (width 0.5) (layer "F.Cu") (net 12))
 (segment (start 127.521204 77.023668) (end 127.521204 88.151204) (width 0.5) (layer "F.Cu") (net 12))
 (segment (start 141.610244 74.300244) (end 138.951204 71.641204) (width 0.5) (layer "F.Cu") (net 12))
 (segment (start 135.280244 95.910244) (end 136.550244 95.910244) (width 0.5) (layer "F.Cu") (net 12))
 (segment (start 133.35 94.020488) (end 133.35 93.98) (width 0.5) (layer "F.Cu") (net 12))
 (segment (start 132.903667 71.641205) (end 127.521204 77.023668) (width 0.5) (layer "F.Cu") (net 12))
 (segment (start 133.35 93.98) (end 135.280244 95.910244) (width 0.5) (layer "F.Cu") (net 12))
 (segment (start 131.460244 95.910244) (end 133.35 94.020488) (width 0.5) (layer "F.Cu") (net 12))
 (segment (start 127.521204 88.151204) (end 133.35 93.98) (width 0.5) (layer "F.Cu") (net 12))
 (segment (start 133.990244 81.920244) (end 137.800244 81.920244) (width 0.5) (layer "F.Cu") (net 1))
 (segment (start 133.990244 81.920244) (end 131.470244 81.920244) (width 0.5) (layer "F.Cu") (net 1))
 (segment (start 137.800244 81.920244) (end 144.170244 88.290244) (width 0.5) (layer "F.Cu") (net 1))
 (segment (start 131.460244 79.390244) (end 133.980244 79.390244) (width 0.5) (layer "F.Cu") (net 13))
 (segment (start 133.990244 79.380244) (end 133.990244 76.840244) (width 0.5) (layer "F.Cu") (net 13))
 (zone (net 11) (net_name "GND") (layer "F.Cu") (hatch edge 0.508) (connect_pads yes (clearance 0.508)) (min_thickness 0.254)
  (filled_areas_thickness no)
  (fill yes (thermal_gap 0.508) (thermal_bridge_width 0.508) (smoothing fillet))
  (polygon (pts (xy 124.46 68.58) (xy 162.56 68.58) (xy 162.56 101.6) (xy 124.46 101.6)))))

